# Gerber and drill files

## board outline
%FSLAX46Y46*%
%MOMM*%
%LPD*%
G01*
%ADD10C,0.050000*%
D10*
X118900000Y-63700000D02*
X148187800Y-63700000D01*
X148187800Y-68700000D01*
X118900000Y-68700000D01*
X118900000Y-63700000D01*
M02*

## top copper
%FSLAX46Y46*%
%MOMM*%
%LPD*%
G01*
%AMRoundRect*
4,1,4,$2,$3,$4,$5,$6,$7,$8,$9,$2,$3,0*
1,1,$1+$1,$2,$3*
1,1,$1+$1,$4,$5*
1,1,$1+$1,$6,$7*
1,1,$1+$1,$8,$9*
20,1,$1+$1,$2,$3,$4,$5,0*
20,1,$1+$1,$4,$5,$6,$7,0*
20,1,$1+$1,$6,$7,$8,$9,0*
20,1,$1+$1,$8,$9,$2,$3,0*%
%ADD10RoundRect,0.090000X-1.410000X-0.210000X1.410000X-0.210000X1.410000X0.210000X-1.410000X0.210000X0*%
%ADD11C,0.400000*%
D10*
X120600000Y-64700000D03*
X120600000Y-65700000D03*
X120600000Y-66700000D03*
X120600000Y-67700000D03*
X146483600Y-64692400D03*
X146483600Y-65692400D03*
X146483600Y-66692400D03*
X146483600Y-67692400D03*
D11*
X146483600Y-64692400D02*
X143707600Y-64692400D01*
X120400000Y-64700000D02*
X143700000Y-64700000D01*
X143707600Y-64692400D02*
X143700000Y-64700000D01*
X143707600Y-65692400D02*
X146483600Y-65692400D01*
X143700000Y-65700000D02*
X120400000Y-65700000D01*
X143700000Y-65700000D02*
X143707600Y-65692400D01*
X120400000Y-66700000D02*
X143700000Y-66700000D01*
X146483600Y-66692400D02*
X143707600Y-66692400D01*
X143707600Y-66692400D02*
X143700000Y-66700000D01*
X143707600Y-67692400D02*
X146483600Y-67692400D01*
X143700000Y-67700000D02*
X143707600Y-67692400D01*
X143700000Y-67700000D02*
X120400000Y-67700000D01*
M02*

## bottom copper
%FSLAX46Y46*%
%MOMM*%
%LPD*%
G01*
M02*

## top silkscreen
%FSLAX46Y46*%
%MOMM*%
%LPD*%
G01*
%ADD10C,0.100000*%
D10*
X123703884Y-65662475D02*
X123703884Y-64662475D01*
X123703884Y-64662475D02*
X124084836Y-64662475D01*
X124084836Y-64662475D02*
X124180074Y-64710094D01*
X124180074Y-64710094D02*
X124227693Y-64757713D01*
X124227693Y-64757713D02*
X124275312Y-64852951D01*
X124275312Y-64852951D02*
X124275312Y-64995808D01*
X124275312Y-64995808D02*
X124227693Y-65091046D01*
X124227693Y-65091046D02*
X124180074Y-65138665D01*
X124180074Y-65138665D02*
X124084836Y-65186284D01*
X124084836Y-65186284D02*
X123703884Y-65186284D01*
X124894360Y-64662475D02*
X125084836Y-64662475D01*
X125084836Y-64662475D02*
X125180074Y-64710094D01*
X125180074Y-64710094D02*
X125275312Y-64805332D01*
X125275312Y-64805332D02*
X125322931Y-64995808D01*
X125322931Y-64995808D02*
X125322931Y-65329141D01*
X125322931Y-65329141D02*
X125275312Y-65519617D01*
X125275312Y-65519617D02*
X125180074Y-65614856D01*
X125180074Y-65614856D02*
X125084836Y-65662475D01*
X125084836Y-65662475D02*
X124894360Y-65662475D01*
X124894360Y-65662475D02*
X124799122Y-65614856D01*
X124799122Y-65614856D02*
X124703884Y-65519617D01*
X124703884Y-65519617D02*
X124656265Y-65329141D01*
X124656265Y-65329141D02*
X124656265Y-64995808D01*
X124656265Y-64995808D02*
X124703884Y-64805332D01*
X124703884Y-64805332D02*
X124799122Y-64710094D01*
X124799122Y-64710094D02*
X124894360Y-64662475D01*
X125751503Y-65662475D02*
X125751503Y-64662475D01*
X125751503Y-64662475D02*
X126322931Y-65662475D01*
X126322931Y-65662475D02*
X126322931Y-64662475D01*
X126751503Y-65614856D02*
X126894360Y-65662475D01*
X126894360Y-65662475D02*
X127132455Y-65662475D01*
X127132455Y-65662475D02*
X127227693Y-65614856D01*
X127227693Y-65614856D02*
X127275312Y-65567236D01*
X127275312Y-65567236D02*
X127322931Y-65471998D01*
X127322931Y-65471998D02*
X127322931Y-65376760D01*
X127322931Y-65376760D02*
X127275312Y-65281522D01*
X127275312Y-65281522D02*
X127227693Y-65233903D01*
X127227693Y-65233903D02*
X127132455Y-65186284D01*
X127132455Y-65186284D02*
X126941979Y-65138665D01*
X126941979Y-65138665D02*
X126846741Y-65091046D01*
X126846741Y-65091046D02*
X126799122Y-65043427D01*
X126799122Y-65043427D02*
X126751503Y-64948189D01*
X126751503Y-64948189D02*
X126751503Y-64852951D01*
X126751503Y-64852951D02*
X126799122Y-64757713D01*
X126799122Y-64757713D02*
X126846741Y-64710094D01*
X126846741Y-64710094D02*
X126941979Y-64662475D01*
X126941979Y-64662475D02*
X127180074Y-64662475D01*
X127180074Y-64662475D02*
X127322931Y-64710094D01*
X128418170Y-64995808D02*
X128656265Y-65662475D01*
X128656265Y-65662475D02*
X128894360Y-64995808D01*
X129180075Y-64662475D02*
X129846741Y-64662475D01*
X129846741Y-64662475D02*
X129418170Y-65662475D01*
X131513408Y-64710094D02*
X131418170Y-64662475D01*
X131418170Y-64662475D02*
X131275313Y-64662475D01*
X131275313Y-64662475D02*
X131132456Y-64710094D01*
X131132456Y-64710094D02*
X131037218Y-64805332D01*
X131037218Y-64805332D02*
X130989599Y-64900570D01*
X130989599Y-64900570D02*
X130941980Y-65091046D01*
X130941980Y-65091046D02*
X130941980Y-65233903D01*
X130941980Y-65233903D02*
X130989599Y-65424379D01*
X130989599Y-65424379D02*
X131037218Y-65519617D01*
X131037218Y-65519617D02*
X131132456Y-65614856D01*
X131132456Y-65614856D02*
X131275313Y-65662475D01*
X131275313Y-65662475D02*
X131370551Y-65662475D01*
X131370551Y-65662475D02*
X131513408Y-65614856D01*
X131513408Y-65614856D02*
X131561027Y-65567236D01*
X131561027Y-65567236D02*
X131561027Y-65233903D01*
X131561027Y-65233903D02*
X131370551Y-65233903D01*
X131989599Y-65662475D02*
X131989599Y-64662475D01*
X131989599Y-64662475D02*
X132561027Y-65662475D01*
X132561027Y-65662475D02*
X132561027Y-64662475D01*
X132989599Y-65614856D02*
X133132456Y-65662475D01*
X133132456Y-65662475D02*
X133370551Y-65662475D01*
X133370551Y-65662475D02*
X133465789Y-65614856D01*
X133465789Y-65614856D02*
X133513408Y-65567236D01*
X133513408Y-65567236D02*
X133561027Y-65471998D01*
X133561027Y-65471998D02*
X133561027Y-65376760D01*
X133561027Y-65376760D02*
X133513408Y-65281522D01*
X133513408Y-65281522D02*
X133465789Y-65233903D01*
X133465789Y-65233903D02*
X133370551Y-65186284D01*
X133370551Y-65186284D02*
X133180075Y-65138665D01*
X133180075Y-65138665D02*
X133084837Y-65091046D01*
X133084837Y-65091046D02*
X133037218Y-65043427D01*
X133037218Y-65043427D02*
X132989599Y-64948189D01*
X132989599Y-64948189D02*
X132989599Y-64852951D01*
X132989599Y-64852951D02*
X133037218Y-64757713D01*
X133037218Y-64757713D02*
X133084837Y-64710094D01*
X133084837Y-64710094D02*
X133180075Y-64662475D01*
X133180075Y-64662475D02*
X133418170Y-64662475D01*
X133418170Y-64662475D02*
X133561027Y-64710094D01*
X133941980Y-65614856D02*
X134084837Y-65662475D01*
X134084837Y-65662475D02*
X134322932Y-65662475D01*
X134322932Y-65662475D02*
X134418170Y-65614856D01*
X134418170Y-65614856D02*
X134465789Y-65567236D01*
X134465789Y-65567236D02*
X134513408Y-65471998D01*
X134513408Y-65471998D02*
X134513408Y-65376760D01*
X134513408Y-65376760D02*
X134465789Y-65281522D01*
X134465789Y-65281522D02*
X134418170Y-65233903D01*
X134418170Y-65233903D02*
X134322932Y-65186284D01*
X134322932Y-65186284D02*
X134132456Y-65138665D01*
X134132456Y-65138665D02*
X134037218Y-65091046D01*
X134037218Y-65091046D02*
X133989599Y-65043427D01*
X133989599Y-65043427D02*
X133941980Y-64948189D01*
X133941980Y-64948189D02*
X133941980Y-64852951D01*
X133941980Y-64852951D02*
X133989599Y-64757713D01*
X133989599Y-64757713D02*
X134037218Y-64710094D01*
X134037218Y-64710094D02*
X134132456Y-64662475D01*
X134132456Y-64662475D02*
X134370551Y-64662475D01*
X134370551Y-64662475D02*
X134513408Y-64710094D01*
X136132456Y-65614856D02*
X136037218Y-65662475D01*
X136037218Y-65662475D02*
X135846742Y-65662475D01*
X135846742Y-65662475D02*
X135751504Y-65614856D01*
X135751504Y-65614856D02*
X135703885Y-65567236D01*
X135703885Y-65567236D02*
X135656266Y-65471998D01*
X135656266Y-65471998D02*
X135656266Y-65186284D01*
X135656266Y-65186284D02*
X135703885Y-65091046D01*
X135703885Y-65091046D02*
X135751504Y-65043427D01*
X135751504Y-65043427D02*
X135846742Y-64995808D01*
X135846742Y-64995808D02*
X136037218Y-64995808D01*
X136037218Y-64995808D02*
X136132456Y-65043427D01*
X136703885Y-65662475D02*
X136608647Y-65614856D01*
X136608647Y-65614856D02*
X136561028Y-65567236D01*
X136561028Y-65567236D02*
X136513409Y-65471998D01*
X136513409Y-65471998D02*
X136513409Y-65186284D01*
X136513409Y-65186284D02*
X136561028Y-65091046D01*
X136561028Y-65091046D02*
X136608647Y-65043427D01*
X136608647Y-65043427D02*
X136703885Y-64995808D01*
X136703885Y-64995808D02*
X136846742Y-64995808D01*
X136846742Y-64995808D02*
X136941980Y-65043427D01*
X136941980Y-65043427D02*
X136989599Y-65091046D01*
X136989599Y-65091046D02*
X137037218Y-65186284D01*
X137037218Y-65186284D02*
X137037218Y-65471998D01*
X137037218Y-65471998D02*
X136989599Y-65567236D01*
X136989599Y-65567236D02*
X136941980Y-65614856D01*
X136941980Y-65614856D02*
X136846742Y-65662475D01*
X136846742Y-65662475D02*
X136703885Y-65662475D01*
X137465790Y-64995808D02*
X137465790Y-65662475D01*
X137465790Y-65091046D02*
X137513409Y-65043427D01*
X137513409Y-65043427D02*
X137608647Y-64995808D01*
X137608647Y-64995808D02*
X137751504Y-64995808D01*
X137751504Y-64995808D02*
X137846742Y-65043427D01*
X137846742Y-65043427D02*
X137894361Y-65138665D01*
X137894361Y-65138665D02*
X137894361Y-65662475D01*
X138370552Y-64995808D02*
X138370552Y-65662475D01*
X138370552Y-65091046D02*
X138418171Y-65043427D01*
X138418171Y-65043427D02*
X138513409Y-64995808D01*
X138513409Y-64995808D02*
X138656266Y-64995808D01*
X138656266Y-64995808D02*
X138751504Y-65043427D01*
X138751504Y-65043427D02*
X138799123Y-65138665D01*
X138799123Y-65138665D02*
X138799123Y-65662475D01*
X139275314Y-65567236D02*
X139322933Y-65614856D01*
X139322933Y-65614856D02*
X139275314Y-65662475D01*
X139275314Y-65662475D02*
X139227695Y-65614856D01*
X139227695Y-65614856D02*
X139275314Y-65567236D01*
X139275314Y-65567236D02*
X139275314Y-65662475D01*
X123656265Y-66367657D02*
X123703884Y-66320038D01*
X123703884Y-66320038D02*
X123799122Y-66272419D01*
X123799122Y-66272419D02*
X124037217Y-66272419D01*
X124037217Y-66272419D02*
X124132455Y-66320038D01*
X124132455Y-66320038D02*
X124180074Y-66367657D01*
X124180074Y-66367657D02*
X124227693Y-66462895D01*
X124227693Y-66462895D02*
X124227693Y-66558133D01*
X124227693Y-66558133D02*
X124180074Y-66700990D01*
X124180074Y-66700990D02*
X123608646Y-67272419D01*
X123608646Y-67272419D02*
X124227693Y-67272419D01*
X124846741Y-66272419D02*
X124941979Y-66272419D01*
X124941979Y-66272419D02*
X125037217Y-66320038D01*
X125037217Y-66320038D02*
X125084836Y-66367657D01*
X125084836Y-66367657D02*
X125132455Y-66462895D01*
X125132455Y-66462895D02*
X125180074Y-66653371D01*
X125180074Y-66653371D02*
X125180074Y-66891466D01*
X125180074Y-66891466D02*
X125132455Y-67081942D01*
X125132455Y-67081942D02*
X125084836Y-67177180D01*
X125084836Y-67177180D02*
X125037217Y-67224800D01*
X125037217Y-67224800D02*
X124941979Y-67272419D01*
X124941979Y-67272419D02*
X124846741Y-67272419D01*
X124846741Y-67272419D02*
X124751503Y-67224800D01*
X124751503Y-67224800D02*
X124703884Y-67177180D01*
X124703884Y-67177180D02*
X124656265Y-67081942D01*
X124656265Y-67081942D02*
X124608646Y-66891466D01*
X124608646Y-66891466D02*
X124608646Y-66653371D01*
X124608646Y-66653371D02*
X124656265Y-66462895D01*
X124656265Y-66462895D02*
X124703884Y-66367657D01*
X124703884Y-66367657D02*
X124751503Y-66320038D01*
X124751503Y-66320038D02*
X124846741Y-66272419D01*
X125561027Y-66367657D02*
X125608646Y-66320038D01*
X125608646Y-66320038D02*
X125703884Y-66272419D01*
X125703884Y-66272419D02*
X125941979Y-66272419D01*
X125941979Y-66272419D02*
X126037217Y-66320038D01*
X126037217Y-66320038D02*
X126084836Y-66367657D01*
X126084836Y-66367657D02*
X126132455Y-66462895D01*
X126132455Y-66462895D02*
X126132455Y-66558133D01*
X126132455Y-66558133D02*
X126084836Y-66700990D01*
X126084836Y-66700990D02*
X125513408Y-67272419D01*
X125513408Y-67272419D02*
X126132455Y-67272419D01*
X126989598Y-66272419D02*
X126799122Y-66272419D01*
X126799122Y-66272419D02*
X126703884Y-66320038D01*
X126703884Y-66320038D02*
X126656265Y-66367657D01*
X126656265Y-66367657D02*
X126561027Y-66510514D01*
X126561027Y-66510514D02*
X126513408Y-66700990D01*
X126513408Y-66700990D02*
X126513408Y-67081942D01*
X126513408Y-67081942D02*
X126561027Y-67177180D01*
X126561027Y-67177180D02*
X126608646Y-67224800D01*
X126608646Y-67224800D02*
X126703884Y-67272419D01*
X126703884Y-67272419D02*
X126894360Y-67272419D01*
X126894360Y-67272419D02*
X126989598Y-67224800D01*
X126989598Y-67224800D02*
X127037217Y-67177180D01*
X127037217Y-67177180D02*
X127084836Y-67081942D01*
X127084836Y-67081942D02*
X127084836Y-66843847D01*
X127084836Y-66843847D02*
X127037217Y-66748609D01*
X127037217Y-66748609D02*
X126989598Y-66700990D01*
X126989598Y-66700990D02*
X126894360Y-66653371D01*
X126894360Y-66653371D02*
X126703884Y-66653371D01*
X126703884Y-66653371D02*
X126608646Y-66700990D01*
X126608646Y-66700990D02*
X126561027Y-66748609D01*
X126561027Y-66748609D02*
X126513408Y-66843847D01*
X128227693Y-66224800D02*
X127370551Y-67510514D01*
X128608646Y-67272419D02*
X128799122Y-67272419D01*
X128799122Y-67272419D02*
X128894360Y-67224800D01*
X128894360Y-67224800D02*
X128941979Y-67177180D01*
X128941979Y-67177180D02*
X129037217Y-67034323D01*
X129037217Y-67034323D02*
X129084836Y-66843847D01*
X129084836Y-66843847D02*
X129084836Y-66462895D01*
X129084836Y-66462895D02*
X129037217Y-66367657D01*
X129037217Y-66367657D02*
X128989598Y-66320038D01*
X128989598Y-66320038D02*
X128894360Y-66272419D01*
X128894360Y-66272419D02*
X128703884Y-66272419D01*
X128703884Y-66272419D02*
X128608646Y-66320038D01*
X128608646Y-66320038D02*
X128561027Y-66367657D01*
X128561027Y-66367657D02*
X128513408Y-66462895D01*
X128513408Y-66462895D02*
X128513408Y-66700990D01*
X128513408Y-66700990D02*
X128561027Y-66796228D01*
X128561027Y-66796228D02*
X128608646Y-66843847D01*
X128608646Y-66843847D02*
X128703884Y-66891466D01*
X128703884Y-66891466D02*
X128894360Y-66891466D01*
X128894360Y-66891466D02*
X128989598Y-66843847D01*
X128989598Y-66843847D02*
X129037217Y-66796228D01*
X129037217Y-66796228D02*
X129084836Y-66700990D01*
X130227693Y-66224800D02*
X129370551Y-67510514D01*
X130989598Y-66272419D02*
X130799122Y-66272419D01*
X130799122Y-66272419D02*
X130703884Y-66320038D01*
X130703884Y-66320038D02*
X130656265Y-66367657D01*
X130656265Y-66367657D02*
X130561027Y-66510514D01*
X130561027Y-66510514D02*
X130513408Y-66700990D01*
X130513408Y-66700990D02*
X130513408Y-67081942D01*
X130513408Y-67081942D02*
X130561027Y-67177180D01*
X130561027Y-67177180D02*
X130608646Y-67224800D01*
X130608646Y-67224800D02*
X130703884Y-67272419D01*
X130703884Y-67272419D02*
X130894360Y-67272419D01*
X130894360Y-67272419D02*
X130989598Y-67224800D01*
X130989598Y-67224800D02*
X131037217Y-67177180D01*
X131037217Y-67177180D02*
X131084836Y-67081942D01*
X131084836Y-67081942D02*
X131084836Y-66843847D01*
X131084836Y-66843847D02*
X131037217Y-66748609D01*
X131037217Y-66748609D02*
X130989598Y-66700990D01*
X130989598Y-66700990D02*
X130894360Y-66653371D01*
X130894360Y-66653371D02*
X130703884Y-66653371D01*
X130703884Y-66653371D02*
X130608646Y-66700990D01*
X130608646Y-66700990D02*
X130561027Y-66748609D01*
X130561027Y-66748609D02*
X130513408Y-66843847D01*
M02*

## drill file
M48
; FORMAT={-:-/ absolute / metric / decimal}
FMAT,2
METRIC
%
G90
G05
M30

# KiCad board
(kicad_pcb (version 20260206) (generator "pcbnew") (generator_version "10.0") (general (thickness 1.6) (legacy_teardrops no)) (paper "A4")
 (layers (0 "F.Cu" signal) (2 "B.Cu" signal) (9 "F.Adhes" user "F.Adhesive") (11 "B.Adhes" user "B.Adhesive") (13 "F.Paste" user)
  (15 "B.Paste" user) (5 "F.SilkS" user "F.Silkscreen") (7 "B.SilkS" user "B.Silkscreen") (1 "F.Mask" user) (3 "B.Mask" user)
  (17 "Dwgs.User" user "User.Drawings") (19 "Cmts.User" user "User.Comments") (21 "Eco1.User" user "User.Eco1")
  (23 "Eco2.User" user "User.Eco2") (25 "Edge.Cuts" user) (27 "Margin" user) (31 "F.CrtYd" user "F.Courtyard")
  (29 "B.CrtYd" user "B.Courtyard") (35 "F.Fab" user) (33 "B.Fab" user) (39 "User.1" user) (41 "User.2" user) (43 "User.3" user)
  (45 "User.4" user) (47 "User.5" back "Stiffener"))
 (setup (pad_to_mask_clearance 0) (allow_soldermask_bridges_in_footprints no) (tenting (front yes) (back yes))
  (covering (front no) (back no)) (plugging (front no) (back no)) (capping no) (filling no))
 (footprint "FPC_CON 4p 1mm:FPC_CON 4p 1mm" (layer "F.Cu") (at 120.6 66.2)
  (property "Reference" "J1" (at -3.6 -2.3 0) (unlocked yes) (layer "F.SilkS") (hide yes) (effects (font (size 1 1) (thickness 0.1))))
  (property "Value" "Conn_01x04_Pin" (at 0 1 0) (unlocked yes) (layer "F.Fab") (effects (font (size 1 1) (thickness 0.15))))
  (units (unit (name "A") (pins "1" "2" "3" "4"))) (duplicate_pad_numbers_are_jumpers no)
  (pad "1" smd roundrect (at 0 -1.5) (size 3 0.6) (layers "F.Cu" "F.Mask" "F.Paste") (roundrect_rratio 0.15) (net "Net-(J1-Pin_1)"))
  (pad "2" smd roundrect (at 0 -0.5) (size 3 0.6) (layers "F.Cu" "F.Mask" "F.Paste") (roundrect_rratio 0.15) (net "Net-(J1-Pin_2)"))
  (pad "3" smd roundrect (at 0 0.5) (size 3 0.6) (layers "F.Cu" "F.Mask" "F.Paste") (roundrect_rratio 0.15) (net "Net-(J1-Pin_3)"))
  (pad "4" smd roundrect (at 0 1.5) (size 3 0.6) (layers "F.Cu" "F.Mask" "F.Paste") (roundrect_rratio 0.15) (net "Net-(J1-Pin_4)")))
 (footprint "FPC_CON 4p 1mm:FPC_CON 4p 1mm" (layer "F.Cu") (at 146.4836 66.1924)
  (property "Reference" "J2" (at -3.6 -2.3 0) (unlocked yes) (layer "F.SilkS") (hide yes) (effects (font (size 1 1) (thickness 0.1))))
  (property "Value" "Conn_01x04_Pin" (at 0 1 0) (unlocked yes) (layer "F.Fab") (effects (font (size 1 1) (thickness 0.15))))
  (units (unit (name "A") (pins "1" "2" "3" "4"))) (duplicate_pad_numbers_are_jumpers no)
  (pad "1" smd roundrect (at 0 -1.5) (size 3 0.6) (layers "F.Cu" "F.Mask" "F.Paste") (roundrect_rratio 0.15) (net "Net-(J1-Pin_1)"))
  (pad "2" smd roundrect (at 0 -0.5) (size 3 0.6) (layers "F.Cu" "F.Mask" "F.Paste") (roundrect_rratio 0.15) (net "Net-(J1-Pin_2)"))
  (pad "3" smd roundrect (at 0 0.5) (size 3 0.6) (layers "F.Cu" "F.Mask" "F.Paste") (roundrect_rratio 0.15) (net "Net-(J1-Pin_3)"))
  (pad "4" smd roundrect (at 0 1.5) (size 3 0.6) (layers "F.Cu" "F.Mask" "F.Paste") (roundrect_rratio 0.15) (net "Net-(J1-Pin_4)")))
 (gr_rect (start 118.9 63.7) (end 148.1878 68.7) (stroke (width 0.05) (type default)) (fill no) (layer "Edge.Cuts"))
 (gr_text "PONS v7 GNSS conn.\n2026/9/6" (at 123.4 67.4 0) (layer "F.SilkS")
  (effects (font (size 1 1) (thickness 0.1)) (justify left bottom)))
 (segment (start 146.4836 64.6924) (end 143.7076 64.6924) (width 0.4) (layer "F.Cu") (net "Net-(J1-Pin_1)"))
 (segment (start 120.4 64.7) (end 143.7 64.7) (width 0.4) (layer "F.Cu") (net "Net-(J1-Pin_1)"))
 (segment (start 143.7076 64.6924) (end 143.7 64.7) (width 0.4) (layer "F.Cu") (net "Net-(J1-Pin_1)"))
 (segment (start 143.7076 65.6924) (end 146.4836 65.6924) (width 0.4) (layer "F.Cu") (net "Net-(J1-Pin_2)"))
 (segment (start 143.7 65.7) (end 120.4 65.7) (width 0.4) (layer "F.Cu") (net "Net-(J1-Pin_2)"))
 (segment (start 143.7 65.7) (end 143.7076 65.6924) (width 0.4) (layer "F.Cu") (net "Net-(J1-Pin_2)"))
 (segment (start 120.4 66.7) (end 143.7 66.7) (width 0.4) (layer "F.Cu") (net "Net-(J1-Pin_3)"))
 (segment (start 146.4836 66.6924) (end 143.7076 66.6924) (width 0.4) (layer "F.Cu") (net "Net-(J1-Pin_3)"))
 (segment (start 143.7076 66.6924) (end 143.7 66.7) (width 0.4) (layer "F.Cu") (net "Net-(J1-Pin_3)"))
 (segment (start 143.7076 67.6924) (end 146.4836 67.6924) (width 0.4) (layer "F.Cu") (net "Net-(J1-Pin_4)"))
 (segment (start 143.7 67.7) (end 143.7076 67.6924) (width 0.4) (layer "F.Cu") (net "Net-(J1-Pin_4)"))
 (segment (start 143.7 67.7) (end 120.4 67.7) (width 0.4) (layer "F.Cu") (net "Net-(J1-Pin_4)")))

